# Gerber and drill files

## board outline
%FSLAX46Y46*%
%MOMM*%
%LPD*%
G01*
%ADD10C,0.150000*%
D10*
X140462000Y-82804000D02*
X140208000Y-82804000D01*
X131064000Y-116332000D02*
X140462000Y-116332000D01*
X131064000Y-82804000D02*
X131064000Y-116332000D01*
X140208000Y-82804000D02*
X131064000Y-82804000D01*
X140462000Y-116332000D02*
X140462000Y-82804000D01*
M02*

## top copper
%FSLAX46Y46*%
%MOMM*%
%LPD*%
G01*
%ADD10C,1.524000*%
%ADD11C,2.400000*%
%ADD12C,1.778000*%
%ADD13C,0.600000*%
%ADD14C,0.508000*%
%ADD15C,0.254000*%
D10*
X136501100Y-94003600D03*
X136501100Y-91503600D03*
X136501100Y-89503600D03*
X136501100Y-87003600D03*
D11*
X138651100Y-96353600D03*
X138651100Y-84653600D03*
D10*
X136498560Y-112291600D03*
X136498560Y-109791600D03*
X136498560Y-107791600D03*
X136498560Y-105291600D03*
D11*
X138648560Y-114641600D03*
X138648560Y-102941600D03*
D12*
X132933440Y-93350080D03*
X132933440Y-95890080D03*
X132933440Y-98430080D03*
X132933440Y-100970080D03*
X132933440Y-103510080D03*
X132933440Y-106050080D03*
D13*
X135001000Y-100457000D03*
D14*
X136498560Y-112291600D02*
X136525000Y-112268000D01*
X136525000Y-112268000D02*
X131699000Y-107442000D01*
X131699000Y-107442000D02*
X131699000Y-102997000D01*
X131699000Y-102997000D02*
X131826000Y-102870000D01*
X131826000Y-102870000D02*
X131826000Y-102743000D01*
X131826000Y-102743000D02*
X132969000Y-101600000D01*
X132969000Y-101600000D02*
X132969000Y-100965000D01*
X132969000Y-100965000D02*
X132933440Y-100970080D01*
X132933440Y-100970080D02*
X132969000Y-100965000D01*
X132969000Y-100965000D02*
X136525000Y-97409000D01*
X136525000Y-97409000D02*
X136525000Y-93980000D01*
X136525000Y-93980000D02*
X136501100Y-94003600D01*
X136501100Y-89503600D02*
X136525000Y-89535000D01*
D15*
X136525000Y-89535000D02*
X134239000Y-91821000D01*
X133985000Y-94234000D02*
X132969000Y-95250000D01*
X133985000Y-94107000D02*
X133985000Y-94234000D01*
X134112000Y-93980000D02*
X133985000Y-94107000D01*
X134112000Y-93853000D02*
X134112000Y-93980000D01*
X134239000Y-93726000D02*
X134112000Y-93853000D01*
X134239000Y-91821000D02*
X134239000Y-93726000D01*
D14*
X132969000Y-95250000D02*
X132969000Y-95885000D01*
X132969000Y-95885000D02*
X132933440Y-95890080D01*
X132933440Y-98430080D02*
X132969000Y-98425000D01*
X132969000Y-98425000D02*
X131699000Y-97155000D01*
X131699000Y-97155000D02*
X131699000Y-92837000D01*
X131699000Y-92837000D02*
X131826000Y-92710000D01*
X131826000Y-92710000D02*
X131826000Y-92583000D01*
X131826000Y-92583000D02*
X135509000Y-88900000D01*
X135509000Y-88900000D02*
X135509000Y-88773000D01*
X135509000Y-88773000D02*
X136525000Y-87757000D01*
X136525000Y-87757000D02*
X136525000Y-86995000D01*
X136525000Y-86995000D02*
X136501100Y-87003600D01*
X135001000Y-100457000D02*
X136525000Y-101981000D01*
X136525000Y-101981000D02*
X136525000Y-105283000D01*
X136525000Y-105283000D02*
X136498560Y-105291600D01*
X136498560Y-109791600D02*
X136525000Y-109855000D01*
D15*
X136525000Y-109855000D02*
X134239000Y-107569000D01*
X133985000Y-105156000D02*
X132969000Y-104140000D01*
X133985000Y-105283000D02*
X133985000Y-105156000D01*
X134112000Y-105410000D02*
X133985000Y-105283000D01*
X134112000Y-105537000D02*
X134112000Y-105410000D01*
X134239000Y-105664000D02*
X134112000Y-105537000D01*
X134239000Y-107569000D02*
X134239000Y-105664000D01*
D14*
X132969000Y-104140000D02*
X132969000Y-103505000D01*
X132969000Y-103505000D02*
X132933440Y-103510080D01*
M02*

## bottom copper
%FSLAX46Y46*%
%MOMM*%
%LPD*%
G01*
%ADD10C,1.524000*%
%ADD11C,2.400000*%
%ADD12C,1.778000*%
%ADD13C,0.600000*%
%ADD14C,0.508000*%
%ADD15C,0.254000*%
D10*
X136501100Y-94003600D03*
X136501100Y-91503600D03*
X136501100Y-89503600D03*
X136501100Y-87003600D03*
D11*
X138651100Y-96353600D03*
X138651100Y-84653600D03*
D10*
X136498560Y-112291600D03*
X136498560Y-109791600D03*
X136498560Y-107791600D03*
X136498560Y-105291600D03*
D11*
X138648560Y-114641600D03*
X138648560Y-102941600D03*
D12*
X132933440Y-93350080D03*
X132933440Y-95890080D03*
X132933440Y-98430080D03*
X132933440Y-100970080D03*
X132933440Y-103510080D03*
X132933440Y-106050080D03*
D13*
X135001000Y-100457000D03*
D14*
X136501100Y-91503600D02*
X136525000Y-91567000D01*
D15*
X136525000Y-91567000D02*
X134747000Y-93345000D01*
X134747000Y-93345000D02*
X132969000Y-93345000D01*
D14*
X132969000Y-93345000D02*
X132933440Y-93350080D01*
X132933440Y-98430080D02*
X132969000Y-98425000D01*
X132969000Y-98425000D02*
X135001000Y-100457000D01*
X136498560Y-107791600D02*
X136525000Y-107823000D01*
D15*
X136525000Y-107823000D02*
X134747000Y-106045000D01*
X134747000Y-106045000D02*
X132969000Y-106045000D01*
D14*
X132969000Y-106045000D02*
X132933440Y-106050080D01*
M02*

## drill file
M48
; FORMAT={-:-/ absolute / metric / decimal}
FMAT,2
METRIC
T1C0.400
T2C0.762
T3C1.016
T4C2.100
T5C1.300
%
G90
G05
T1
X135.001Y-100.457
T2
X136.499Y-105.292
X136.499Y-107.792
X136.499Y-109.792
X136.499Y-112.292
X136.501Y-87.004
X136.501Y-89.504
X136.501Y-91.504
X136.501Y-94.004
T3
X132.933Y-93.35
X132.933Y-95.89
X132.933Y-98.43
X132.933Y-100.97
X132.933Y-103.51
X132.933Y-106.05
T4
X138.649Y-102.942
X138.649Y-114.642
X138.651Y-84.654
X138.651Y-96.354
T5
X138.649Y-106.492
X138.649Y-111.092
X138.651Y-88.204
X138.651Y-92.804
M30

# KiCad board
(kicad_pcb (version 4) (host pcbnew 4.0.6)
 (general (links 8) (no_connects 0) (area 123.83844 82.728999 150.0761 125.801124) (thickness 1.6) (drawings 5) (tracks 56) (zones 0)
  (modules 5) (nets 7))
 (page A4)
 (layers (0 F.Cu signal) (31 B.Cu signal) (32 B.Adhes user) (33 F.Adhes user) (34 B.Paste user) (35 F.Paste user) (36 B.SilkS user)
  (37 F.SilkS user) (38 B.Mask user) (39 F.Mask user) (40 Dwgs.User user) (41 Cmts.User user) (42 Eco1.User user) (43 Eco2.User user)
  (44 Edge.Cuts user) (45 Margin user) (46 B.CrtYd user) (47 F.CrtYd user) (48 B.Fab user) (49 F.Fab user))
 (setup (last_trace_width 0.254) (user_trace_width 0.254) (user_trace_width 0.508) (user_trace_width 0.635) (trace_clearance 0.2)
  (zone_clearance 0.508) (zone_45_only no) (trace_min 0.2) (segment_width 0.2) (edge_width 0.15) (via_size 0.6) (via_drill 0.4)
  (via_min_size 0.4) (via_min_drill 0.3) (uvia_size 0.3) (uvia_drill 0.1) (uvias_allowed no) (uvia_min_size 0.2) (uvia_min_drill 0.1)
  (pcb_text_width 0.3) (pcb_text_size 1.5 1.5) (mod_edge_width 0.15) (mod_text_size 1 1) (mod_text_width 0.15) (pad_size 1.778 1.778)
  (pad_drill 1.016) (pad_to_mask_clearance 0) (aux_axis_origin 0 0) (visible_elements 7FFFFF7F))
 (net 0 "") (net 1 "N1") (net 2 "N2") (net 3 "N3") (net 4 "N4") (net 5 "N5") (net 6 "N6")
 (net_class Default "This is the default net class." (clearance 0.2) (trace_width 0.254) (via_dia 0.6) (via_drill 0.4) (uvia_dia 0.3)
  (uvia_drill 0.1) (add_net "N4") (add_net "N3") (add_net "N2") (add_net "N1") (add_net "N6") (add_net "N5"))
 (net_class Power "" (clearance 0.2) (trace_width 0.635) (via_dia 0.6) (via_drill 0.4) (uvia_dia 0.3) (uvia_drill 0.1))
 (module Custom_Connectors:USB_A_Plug (layer F.Cu) (at 148.5011 105.0036 90)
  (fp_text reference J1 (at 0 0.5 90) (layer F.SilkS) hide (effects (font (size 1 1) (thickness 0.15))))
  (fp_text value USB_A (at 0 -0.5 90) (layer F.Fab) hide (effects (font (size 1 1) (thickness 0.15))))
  (pad 4 thru_hole circle (at 11 -12 90) (size 1.524 1.524) (drill 0.762) (layers *.Cu *.Mask) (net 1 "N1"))
  (pad 3 thru_hole circle (at 13.5 -12 90) (size 1.524 1.524) (drill 0.762) (layers *.Cu *.Mask) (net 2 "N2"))
  (pad 2 thru_hole circle (at 15.5 -12 90) (size 1.524 1.524) (drill 0.762) (layers *.Cu *.Mask) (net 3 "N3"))
  (pad 1 thru_hole circle (at 18 -12 90) (size 1.524 1.524) (drill 0.762) (layers *.Cu *.Mask) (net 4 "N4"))
  (pad "" np_thru_hole circle (at 12.2 -9.85 90) (size 1.3 1.3) (drill 1.3) (layers *.Cu *.Mask))
  (pad "" np_thru_hole circle (at 16.8 -9.85 90) (size 1.3 1.3) (drill 1.3) (layers *.Cu *.Mask))
  (pad 7 thru_hole circle (at 8.65 -9.85 90) (size 2.4 2.4) (drill 2.1) (layers *.Cu *.Mask))
  (pad 6 thru_hole circle (at 20.35 -9.85 90) (size 2.4 2.4) (drill 2.1) (layers *.Cu *.Mask)))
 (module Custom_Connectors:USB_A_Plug (layer F.Cu) (at 148.49856 123.2916 90)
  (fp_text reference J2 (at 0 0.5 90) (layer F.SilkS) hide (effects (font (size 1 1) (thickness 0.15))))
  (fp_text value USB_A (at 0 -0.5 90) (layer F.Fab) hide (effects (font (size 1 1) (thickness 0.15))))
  (pad 4 thru_hole circle (at 11 -12 90) (size 1.524 1.524) (drill 0.762) (layers *.Cu *.Mask) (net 1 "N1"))
  (pad 3 thru_hole circle (at 13.5 -12 90) (size 1.524 1.524) (drill 0.762) (layers *.Cu *.Mask) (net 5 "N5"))
  (pad 2 thru_hole circle (at 15.5 -12 90) (size 1.524 1.524) (drill 0.762) (layers *.Cu *.Mask) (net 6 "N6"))
  (pad 1 thru_hole circle (at 18 -12 90) (size 1.524 1.524) (drill 0.762) (layers *.Cu *.Mask) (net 4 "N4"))
  (pad "" np_thru_hole circle (at 12.2 -9.85 90) (size 1.3 1.3) (drill 1.3) (layers *.Cu *.Mask))
  (pad "" np_thru_hole circle (at 16.8 -9.85 90) (size 1.3 1.3) (drill 1.3) (layers *.Cu *.Mask))
  (pad 7 thru_hole circle (at 8.65 -9.85 90) (size 2.4 2.4) (drill 2.1) (layers *.Cu *.Mask))
  (pad 6 thru_hole circle (at 20.35 -9.85 90) (size 2.4 2.4) (drill 2.1) (layers *.Cu *.Mask)))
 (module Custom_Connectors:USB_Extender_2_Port (layer F.Cu) (at 125.31344 88.27008 270)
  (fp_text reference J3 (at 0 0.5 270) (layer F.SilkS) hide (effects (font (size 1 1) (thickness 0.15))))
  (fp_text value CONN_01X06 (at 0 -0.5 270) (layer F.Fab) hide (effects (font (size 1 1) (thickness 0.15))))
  (pad 1 thru_hole circle (at 5.08 -7.62 270) (size 1.778 1.778) (drill 1.016) (layers *.Cu *.Mask) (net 2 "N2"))
  (pad 2 thru_hole circle (at 7.62 -7.62 270) (size 1.778 1.778) (drill 1.016) (layers *.Cu *.Mask) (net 3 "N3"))
  (pad 3 thru_hole circle (at 10.16 -7.62 270) (size 1.778 1.778) (drill 1.016) (layers *.Cu *.Mask) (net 4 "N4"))
  (pad 4 thru_hole circle (at 12.7 -7.62 270) (size 1.778 1.778) (drill 1.016) (layers *.Cu *.Mask) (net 1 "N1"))
  (pad 5 thru_hole circle (at 15.24 -7.62 270) (size 1.778 1.778) (drill 1.016) (layers *.Cu *.Mask) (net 5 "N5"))
  (pad 6 thru_hole circle (at 17.78 -7.62 270) (size 1.778 1.778) (drill 1.016) (layers *.Cu *.Mask) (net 6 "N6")))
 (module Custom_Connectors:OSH (layer F.Cu) (at 133.35 113.538 270)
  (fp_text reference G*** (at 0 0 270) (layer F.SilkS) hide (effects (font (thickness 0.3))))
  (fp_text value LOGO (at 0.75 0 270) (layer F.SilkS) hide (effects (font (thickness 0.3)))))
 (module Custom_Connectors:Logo (layer F.Cu) (at 133.35 86.106 270)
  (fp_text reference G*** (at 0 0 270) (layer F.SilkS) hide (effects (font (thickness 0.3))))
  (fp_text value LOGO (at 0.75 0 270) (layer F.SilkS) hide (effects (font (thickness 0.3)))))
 (gr_line (start 140.462 82.804) (end 140.208 82.804) (angle 90) (layer Edge.Cuts) (width 0.15))
 (gr_line (start 131.064 116.332) (end 140.462 116.332) (angle 90) (layer Edge.Cuts) (width 0.15))
 (gr_line (start 131.064 82.804) (end 131.064 116.332) (angle 90) (layer Edge.Cuts) (width 0.15))
 (gr_line (start 140.208 82.804) (end 131.064 82.804) (angle 90) (layer Edge.Cuts) (width 0.15))
 (gr_line (start 140.462 116.332) (end 140.462 82.804) (angle 90) (layer Edge.Cuts) (width 0.15))
 (segment (start 136.49856 112.2916) (end 136.525 112.268) (width 0.508) (layer F.Cu) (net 1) (status 80000))
 (segment (start 136.525 112.268) (end 131.699 107.442) (width 0.508) (layer F.Cu) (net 1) (status 80000))
 (segment (start 131.699 107.442) (end 131.699 102.997) (width 0.508) (layer F.Cu) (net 1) (status 80000))
 (segment (start 131.699 102.997) (end 131.826 102.87) (width 0.508) (layer F.Cu) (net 1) (status 80000))
 (segment (start 131.826 102.87) (end 131.826 102.743) (width 0.508) (layer F.Cu) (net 1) (status 80000))
 (segment (start 131.826 102.743) (end 132.969 101.6) (width 0.508) (layer F.Cu) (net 1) (status 80000))
 (segment (start 132.969 101.6) (end 132.969 100.965) (width 0.508) (layer F.Cu) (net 1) (status 80000))
 (segment (start 132.969 100.965) (end 132.93344 100.97008) (width 0.508) (layer F.Cu) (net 1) (status 80000))
 (segment (start 132.93344 100.97008) (end 132.969 100.965) (width 0.508) (layer F.Cu) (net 1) (status 80000))
 (segment (start 132.969 100.965) (end 136.525 97.409) (width 0.508) (layer F.Cu) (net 1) (status 80000))
 (segment (start 136.525 97.409) (end 136.525 93.98) (width 0.508) (layer F.Cu) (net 1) (status 80000))
 (segment (start 136.525 93.98) (end 136.5011 94.0036) (width 0.508) (layer F.Cu) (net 1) (status 80000))
 (segment (start 136.5011 91.5036) (end 136.525 91.567) (width 0.508) (layer B.Cu) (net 2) (status 80000))
 (segment (start 136.525 91.567) (end 134.747 93.345) (width 0.254) (layer B.Cu) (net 2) (status 80000))
 (segment (start 134.747 93.345) (end 132.969 93.345) (width 0.254) (layer B.Cu) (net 2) (status 80000))
 (segment (start 132.969 93.345) (end 132.93344 93.35008) (width 0.508) (layer B.Cu) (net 2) (status 80000))
 (segment (start 136.5011 89.5036) (end 136.525 89.535) (width 0.508) (layer F.Cu) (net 3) (status 80000))
 (segment (start 136.525 89.535) (end 134.239 91.821) (width 0.254) (layer F.Cu) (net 3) (status 80000))
 (segment (start 133.985 94.234) (end 132.969 95.25) (width 0.254) (layer F.Cu) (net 3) (status 80000))
 (segment (start 133.985 94.107) (end 133.985 94.234) (width 0.254) (layer F.Cu) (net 3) (status 80000))
 (segment (start 134.112 93.98) (end 133.985 94.107) (width 0.254) (layer F.Cu) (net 3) (status 80000))
 (segment (start 134.112 93.853) (end 134.112 93.98) (width 0.254) (layer F.Cu) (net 3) (status 80000))
 (segment (start 134.239 93.726) (end 134.112 93.853) (width 0.254) (layer F.Cu) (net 3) (status 80000))
 (segment (start 134.239 91.821) (end 134.239 93.726) (width 0.254) (layer F.Cu) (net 3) (status 80000))
 (segment (start 132.969 95.25) (end 132.969 95.885) (width 0.508) (layer F.Cu) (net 3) (status 80000))
 (segment (start 132.969 95.885) (end 132.93344 95.89008) (width 0.508) (layer F.Cu) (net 3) (status 80000))
 (segment (start 132.93344 98.43008) (end 132.969 98.425) (width 0.508) (layer F.Cu) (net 4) (status 80000))
 (segment (start 132.969 98.425) (end 131.699 97.155) (width 0.508) (layer F.Cu) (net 4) (status 80000))
 (segment (start 131.699 97.155) (end 131.699 92.837) (width 0.508) (layer F.Cu) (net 4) (status 80000))
 (segment (start 131.699 92.837) (end 131.826 92.71) (width 0.508) (layer F.Cu) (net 4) (status 80000))
 (segment (start 131.826 92.71) (end 131.826 92.583) (width 0.508) (layer F.Cu) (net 4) (status 80000))
 (segment (start 131.826 92.583) (end 135.509 88.9) (width 0.508) (layer F.Cu) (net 4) (status 80000))
 (segment (start 135.509 88.9) (end 135.509 88.773) (width 0.508) (layer F.Cu) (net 4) (status 80000))
 (segment (start 135.509 88.773) (end 136.525 87.757) (width 0.508) (layer F.Cu) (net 4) (status 80000))
 (segment (start 136.525 87.757) (end 136.525 86.995) (width 0.508) (layer F.Cu) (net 4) (status 80000))
 (segment (start 136.525 86.995) (end 136.5011 87.0036) (width 0.508) (layer F.Cu) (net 4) (status 80000))
 (segment (start 132.93344 98.43008) (end 132.969 98.425) (width 0.508) (layer B.Cu) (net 4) (status 80000))
 (segment (start 132.969 98.425) (end 135.001 100.457) (width 0.508) (layer B.Cu) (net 4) (status 80000))
 (via (at 135.001 100.457) (size 0.6) (layers F.Cu B.Cu) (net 4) (status 80000))
 (segment (start 135.001 100.457) (end 136.525 101.981) (width 0.508) (layer F.Cu) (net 4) (status 80000))
 (segment (start 136.525 101.981) (end 136.525 105.283) (width 0.508) (layer F.Cu) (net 4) (status 80000))
 (segment (start 136.525 105.283) (end 136.49856 105.2916) (width 0.508) (layer F.Cu) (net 4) (status 80000))
 (segment (start 136.49856 109.7916) (end 136.525 109.855) (width 0.508) (layer F.Cu) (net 5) (status 80000))
 (segment (start 136.525 109.855) (end 134.239 107.569) (width 0.254) (layer F.Cu) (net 5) (status 80000))
 (segment (start 133.985 105.156) (end 132.969 104.14) (width 0.254) (layer F.Cu) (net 5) (status 80000))
 (segment (start 133.985 105.283) (end 133.985 105.156) (width 0.254) (layer F.Cu) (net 5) (status 80000))
 (segment (start 134.112 105.41) (end 133.985 105.283) (width 0.254) (layer F.Cu) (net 5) (status 80000))
 (segment (start 134.112 105.537) (end 134.112 105.41) (width 0.254) (layer F.Cu) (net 5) (status 80000))
 (segment (start 134.239 105.664) (end 134.112 105.537) (width 0.254) (layer F.Cu) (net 5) (status 80000))
 (segment (start 134.239 107.569) (end 134.239 105.664) (width 0.254) (layer F.Cu) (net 5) (status 80000))
 (segment (start 132.969 104.14) (end 132.969 103.505) (width 0.508) (layer F.Cu) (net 5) (status 80000))
 (segment (start 132.969 103.505) (end 132.93344 103.51008) (width 0.508) (layer F.Cu) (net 5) (status 80000))
 (segment (start 136.49856 107.7916) (end 136.525 107.823) (width 0.508) (layer B.Cu) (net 6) (status 80000))
 (segment (start 136.525 107.823) (end 134.747 106.045) (width 0.254) (layer B.Cu) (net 6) (status 80000))
 (segment (start 134.747 106.045) (end 132.969 106.045) (width 0.254) (layer B.Cu) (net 6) (status 80000))
 (segment (start 132.969 106.045) (end 132.93344 106.05008) (width 0.508) (layer B.Cu) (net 6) (status 80000)))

